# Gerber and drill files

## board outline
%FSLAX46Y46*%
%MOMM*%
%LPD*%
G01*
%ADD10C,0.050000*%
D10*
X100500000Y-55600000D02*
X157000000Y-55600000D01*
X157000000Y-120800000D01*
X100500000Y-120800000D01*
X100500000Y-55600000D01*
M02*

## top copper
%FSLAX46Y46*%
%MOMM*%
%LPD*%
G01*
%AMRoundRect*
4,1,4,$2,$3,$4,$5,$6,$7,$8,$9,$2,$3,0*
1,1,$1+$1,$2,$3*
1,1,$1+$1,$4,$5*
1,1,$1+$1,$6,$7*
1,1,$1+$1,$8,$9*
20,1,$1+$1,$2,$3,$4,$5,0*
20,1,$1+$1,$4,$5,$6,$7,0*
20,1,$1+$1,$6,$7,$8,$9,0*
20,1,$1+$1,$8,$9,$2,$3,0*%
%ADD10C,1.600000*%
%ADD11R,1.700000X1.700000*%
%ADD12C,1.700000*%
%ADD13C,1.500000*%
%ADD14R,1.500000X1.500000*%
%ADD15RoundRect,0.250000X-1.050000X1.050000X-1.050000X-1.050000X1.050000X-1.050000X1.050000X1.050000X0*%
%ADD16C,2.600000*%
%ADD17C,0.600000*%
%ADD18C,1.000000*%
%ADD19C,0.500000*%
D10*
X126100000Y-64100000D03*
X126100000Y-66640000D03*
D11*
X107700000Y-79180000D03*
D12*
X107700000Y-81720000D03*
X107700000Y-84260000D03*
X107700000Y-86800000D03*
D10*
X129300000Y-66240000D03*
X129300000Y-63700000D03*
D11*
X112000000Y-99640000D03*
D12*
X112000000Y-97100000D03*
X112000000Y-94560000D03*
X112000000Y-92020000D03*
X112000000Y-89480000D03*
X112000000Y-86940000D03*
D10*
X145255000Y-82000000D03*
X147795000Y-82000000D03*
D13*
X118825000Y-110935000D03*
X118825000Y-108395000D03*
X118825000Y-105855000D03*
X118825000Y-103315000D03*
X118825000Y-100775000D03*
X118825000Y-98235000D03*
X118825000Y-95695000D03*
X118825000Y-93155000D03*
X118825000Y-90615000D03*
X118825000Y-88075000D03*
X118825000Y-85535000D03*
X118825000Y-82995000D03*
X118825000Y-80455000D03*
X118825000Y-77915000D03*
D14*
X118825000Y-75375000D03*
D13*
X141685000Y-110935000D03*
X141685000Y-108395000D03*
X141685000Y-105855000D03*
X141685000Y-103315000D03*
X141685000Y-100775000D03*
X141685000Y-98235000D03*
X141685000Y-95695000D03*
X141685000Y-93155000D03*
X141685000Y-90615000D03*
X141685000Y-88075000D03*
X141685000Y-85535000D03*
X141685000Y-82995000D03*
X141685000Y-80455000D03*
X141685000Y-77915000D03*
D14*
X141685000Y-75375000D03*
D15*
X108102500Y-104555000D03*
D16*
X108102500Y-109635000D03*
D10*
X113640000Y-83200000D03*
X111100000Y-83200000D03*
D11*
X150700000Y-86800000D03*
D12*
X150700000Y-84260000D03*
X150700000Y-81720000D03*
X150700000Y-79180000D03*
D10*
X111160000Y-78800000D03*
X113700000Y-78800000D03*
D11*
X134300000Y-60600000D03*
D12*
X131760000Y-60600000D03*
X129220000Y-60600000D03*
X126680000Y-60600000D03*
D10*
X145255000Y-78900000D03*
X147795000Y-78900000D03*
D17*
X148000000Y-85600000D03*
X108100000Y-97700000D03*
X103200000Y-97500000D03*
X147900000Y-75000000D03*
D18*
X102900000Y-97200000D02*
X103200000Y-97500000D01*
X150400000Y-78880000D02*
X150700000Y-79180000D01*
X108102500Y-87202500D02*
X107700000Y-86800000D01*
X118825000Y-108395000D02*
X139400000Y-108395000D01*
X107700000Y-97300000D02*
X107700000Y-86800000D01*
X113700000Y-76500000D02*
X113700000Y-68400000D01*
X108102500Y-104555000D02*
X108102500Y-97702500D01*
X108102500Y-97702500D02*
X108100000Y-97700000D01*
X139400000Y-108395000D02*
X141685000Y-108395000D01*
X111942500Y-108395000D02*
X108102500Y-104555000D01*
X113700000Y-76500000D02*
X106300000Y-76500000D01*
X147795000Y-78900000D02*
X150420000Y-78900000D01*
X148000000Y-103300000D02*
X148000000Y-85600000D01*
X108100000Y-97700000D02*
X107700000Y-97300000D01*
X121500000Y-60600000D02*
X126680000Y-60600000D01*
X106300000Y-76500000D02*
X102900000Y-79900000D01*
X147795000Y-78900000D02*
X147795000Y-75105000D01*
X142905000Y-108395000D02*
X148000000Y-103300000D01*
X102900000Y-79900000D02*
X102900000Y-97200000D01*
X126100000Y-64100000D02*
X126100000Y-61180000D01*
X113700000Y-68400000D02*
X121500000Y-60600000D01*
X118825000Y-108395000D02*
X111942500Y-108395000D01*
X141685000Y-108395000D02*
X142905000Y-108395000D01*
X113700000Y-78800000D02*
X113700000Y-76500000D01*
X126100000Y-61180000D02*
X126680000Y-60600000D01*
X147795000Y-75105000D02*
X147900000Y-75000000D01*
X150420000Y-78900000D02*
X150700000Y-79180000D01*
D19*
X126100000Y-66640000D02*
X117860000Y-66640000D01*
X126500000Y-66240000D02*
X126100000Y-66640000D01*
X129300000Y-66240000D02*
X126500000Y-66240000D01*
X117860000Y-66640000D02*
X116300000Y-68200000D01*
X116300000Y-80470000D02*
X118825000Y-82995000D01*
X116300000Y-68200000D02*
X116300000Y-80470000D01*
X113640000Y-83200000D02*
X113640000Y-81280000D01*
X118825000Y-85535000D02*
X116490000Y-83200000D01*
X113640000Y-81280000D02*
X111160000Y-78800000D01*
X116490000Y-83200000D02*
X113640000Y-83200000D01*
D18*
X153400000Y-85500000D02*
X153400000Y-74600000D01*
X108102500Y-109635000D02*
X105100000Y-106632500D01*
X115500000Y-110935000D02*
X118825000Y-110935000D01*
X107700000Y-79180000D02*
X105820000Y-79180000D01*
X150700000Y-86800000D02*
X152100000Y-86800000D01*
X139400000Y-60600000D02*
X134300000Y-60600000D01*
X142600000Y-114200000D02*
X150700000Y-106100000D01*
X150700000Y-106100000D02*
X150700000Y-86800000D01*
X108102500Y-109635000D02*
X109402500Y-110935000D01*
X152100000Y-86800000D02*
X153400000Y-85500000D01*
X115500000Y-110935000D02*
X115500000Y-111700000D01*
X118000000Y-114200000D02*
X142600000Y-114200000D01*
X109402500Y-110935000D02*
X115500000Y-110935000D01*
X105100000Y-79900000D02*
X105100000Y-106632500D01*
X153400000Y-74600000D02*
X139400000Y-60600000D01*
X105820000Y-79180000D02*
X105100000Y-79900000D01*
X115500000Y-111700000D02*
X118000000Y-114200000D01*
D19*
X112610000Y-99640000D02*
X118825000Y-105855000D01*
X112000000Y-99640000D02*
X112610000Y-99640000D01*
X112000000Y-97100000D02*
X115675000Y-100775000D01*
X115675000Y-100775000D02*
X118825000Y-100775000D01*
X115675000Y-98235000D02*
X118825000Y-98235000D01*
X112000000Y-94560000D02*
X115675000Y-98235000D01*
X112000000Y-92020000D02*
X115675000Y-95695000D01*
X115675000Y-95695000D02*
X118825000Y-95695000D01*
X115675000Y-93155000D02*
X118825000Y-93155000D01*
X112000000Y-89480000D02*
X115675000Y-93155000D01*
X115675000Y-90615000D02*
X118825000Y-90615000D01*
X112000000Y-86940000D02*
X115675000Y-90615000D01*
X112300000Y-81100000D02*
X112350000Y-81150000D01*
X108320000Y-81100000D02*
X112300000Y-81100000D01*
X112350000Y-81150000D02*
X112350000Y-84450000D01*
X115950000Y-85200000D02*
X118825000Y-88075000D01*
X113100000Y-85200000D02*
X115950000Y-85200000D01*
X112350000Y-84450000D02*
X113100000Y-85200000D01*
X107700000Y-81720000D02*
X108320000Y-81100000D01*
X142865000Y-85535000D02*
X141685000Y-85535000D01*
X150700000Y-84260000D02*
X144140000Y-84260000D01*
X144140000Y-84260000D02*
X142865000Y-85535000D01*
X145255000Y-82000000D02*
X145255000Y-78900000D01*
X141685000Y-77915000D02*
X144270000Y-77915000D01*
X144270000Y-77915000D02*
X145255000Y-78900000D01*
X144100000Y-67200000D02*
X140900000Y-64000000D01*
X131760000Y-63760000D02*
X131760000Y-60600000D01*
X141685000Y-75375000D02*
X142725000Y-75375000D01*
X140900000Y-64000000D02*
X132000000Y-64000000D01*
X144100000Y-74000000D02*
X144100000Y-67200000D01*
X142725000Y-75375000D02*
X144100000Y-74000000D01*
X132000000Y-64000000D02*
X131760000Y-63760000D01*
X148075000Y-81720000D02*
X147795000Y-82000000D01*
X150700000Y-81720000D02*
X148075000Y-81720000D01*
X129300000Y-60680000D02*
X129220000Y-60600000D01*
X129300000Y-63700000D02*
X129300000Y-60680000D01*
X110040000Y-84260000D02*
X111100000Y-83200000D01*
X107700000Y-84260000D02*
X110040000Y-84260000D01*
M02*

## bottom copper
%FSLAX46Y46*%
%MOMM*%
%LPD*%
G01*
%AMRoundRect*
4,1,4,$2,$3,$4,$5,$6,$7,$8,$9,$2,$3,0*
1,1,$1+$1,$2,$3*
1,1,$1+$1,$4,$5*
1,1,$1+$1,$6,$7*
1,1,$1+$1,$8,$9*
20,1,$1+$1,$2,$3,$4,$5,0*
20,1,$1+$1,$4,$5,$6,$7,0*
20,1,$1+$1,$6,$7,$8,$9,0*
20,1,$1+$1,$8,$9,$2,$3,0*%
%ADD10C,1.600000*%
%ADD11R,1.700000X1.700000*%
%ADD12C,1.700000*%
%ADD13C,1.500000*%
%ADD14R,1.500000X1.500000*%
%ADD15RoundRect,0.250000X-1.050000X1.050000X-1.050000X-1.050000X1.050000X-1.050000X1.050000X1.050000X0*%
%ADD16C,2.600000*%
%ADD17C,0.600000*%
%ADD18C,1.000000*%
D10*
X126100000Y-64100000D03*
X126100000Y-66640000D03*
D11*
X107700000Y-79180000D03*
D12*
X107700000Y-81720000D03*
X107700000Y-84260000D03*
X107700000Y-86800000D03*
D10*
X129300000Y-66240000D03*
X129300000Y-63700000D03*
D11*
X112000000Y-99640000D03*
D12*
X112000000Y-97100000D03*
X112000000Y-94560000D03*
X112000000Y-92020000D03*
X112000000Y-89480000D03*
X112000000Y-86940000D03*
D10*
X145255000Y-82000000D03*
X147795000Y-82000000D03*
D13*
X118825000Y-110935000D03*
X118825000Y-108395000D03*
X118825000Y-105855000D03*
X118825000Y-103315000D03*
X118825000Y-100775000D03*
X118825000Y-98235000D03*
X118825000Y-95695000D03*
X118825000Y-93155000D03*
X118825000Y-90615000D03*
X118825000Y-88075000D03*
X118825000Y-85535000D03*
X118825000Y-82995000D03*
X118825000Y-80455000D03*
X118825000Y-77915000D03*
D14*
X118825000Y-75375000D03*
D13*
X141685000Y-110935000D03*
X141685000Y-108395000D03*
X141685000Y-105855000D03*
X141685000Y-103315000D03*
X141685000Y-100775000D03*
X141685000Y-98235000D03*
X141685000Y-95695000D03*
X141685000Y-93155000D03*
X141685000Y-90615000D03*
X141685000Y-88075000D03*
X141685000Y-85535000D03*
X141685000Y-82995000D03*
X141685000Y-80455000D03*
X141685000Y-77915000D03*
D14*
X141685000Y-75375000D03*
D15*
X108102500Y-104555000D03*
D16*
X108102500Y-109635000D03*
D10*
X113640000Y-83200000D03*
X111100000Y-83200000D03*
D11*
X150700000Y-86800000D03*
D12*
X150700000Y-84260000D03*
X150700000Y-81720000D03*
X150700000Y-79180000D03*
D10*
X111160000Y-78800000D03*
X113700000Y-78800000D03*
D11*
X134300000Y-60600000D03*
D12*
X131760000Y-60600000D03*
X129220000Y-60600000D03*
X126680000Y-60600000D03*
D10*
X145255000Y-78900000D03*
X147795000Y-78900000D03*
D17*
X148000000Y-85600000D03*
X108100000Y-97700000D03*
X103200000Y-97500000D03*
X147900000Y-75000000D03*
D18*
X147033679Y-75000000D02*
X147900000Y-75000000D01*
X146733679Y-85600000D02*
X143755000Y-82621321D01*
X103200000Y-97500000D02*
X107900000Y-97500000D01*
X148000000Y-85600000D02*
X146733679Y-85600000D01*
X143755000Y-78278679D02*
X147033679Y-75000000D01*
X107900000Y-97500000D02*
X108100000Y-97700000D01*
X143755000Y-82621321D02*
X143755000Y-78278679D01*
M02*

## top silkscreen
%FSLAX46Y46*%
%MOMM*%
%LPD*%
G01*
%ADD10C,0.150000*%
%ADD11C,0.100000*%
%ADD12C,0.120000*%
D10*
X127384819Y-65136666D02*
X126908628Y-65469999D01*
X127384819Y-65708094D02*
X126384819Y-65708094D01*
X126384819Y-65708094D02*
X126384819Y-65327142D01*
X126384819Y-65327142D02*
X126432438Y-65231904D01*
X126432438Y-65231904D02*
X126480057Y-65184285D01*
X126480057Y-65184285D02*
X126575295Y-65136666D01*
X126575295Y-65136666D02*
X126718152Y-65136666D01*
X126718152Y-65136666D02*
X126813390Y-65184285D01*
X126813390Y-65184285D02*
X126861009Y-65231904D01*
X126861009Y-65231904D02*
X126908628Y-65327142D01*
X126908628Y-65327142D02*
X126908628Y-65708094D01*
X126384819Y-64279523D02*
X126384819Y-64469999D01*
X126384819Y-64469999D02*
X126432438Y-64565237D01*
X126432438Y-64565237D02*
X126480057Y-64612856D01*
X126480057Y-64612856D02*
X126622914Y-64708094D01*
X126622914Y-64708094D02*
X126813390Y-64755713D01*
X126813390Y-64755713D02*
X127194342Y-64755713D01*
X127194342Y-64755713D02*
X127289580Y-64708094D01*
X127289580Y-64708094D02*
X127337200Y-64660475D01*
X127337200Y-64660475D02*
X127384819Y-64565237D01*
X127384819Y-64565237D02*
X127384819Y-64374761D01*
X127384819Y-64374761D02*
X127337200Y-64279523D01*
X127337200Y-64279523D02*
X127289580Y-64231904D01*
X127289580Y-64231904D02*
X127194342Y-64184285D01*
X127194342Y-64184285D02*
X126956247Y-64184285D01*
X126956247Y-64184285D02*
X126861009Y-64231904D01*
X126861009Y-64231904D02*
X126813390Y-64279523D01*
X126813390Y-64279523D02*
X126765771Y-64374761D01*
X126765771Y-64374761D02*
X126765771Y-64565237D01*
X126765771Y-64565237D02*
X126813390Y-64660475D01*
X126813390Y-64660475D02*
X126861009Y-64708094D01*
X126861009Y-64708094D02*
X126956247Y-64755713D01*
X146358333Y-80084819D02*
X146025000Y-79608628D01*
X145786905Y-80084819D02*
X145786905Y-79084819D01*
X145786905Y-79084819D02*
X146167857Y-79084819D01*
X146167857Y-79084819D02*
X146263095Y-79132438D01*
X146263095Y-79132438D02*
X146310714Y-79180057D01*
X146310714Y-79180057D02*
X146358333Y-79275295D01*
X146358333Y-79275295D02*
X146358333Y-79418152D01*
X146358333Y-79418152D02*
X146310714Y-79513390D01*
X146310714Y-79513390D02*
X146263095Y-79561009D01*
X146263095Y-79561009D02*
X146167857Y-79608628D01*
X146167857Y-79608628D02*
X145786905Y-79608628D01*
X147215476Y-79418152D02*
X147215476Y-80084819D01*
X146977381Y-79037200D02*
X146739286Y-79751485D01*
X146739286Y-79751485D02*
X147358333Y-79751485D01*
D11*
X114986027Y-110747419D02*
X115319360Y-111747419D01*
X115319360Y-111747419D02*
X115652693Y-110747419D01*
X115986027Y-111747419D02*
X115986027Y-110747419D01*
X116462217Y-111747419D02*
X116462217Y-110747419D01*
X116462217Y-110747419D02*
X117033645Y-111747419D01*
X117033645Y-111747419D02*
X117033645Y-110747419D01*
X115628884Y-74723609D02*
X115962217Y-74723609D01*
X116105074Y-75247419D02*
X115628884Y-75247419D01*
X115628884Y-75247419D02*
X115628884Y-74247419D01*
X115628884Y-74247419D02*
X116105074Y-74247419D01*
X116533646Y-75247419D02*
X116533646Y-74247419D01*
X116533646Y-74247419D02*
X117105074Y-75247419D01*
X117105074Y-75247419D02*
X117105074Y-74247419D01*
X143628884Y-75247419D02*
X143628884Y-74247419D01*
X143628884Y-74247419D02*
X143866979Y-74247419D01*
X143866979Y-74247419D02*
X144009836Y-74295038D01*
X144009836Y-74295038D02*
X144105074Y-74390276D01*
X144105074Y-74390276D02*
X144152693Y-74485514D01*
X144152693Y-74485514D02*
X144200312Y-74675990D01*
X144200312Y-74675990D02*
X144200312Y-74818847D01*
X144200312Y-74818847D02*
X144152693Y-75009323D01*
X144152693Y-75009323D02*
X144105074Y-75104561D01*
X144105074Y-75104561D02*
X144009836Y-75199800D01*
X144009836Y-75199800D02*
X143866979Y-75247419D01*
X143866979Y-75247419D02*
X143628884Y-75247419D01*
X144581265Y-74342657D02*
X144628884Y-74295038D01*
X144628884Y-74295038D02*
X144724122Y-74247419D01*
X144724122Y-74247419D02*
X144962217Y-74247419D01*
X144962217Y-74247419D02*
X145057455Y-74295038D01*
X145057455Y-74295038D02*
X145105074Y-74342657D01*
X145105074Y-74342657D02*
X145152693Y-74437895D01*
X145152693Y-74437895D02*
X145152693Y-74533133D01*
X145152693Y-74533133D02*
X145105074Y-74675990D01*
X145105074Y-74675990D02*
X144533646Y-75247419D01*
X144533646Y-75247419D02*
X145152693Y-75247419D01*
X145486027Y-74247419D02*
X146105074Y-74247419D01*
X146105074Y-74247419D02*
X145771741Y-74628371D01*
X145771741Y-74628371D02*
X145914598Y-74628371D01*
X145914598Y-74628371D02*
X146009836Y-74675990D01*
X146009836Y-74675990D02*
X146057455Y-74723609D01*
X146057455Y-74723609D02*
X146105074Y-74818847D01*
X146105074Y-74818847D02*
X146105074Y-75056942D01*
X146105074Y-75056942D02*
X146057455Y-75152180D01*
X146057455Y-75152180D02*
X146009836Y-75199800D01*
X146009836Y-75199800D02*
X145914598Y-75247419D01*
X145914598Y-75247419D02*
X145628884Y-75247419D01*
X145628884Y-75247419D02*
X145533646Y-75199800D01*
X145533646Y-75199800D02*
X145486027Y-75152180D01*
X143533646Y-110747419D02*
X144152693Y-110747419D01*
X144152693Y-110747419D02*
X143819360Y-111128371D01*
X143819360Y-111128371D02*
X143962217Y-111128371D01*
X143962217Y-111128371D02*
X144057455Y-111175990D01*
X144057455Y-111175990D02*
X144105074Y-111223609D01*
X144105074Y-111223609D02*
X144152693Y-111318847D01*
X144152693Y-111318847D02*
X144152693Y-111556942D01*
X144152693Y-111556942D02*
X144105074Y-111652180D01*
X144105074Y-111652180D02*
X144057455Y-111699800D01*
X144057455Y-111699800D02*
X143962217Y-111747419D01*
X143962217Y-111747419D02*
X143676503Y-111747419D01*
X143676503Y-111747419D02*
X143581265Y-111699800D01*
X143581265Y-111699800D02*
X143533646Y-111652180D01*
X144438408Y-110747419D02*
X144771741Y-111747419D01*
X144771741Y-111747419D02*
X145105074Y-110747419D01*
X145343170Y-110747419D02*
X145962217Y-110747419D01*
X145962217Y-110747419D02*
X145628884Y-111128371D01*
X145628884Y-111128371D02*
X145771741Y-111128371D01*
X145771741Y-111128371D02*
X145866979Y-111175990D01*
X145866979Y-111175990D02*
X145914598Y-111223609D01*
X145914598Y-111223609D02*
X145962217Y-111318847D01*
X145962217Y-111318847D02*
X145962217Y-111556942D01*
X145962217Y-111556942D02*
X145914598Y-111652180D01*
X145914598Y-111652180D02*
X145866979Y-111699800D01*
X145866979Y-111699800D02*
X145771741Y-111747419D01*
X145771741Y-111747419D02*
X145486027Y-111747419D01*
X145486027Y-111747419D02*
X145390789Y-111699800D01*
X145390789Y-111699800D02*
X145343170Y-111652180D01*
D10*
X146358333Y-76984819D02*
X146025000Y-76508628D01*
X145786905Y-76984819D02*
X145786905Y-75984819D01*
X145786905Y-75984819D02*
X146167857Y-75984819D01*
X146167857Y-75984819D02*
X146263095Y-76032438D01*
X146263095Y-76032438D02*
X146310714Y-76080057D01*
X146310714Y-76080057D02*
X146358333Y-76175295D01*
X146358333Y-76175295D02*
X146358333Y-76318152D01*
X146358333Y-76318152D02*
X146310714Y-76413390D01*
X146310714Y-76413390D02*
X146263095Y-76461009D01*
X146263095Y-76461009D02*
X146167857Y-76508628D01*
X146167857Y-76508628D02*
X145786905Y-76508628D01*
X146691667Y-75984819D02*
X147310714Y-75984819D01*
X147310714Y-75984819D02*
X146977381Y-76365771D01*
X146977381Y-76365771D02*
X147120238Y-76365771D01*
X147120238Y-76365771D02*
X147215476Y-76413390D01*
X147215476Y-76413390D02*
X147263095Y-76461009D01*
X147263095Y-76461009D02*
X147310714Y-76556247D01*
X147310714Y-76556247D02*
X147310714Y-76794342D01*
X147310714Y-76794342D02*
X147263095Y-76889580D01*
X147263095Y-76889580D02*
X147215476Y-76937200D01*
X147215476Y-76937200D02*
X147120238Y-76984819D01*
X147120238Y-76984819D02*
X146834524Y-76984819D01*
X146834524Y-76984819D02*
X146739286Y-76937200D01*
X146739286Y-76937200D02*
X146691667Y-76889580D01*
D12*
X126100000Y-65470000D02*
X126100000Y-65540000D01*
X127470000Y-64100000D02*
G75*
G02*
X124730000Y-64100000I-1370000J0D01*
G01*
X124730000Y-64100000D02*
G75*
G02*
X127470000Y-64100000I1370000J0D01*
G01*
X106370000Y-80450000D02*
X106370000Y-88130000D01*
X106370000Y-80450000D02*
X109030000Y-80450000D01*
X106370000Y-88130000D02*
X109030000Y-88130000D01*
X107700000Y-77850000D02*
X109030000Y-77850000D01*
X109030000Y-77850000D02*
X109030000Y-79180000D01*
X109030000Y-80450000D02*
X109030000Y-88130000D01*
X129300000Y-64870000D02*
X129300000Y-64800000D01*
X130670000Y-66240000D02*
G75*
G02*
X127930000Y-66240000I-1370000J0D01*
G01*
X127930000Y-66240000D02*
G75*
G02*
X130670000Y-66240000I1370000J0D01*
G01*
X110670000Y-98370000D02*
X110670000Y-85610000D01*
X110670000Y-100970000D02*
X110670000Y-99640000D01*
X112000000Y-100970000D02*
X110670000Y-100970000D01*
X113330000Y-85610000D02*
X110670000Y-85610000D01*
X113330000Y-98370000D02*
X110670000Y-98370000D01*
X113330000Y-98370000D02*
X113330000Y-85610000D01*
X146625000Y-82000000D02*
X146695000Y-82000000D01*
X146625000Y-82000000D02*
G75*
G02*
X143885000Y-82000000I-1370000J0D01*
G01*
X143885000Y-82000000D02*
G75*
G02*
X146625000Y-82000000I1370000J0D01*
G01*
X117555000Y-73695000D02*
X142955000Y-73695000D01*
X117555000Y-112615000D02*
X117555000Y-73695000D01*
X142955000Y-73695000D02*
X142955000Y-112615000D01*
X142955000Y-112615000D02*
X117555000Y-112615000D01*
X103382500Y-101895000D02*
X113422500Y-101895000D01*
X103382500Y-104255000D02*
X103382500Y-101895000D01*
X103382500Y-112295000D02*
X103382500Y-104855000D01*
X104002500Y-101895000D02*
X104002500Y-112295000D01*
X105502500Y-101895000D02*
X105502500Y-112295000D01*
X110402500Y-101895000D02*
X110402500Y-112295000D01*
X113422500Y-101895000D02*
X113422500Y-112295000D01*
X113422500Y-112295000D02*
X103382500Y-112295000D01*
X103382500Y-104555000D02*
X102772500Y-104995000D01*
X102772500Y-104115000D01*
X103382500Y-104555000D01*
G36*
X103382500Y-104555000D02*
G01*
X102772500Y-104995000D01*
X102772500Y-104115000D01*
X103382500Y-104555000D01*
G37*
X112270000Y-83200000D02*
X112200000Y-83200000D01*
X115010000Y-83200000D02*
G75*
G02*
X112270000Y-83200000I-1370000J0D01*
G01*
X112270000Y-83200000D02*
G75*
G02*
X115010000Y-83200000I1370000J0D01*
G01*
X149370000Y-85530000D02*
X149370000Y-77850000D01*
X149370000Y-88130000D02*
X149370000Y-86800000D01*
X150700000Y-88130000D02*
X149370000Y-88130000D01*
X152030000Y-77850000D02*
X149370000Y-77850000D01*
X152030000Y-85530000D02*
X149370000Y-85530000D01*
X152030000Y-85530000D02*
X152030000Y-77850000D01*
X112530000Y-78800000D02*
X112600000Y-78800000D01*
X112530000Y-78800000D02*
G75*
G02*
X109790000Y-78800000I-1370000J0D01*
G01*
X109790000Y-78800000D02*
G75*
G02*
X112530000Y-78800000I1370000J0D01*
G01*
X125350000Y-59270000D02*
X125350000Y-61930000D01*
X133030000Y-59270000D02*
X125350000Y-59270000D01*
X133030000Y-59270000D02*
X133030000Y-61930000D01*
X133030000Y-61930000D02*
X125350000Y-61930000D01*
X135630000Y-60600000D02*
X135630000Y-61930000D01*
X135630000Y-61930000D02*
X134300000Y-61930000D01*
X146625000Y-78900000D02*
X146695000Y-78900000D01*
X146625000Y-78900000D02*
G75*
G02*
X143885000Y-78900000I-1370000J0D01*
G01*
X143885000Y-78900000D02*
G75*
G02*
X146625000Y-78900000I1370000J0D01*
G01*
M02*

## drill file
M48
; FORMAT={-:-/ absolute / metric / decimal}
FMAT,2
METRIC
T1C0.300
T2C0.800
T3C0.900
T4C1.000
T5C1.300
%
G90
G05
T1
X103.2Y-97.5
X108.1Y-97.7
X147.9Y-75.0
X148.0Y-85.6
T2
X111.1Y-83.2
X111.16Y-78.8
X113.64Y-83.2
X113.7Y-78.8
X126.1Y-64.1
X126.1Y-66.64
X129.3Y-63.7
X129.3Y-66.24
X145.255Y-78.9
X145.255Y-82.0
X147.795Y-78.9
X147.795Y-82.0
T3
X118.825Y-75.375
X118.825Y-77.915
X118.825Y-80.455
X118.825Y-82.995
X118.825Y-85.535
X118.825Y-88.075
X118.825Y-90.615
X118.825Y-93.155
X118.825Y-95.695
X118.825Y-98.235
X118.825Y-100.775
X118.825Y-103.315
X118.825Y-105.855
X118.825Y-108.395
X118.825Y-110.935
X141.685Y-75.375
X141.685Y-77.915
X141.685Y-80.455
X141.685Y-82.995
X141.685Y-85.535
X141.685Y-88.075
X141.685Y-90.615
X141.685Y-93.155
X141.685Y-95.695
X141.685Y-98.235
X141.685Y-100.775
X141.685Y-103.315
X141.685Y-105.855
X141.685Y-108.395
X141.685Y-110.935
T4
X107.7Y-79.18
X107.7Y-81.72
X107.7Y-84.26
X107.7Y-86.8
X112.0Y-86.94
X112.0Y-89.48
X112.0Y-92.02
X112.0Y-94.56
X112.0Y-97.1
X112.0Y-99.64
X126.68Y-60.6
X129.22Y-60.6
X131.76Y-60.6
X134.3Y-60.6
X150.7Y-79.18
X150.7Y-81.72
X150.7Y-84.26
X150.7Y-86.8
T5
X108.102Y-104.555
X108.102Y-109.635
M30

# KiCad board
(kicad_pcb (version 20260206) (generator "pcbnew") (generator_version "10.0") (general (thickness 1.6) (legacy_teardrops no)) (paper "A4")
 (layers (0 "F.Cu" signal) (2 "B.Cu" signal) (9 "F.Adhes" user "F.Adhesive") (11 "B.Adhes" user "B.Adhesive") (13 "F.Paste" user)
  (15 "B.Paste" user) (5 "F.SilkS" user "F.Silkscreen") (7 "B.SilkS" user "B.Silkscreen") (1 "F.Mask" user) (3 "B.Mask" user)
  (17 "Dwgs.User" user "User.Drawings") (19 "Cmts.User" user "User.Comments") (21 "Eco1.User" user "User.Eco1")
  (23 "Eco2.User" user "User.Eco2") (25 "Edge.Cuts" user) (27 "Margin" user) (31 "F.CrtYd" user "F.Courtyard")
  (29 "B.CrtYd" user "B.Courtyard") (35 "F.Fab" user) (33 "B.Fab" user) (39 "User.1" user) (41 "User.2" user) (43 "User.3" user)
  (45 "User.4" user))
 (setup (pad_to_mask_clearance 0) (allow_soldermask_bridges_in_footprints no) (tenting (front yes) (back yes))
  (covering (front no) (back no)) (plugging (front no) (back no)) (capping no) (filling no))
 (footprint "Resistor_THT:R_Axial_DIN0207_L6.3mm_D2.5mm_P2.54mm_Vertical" (layer "F.Cu") (at 126.1 64.1 -90)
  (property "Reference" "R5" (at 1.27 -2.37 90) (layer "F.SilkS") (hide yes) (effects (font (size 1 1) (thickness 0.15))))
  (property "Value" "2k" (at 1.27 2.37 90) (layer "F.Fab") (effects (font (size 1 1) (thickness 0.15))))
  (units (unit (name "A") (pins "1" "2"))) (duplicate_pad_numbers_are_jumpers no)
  (fp_line (start 1.37 0) (end 1.44 0) (stroke (width 0.12) (type solid)) (layer "F.SilkS"))
  (fp_circle (center 0 0) (end 1.37 0) (stroke (width 0.12) (type solid)) (fill no) (layer "F.SilkS"))
  (pad "1" thru_hole circle (at 0 0 270) (size 1.6 1.6) (drill 0.8) (layers "*.Cu" "*.Mask") (remove_unused_layers no) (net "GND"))
  (pad "2" thru_hole circle (at 2.54 0 270) (size 1.6 1.6) (drill 0.8) (layers "*.Cu" "*.Mask") (remove_unused_layers no)
   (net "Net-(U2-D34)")))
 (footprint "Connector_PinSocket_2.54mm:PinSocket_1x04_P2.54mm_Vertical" (layer "F.Cu") (at 107.7 79.18)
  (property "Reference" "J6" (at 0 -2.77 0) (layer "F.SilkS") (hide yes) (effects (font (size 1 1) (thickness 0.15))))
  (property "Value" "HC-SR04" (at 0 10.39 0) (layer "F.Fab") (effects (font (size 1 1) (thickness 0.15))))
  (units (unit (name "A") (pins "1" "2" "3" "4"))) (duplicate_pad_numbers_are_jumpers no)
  (fp_line (start -1.33 1.27) (end -1.33 8.95) (stroke (width 0.12) (type solid)) (layer "F.SilkS"))
  (fp_line (start -1.33 1.27) (end 1.33 1.27) (stroke (width 0.12) (type solid)) (layer "F.SilkS"))
  (fp_line (start -1.33 8.95) (end 1.33 8.95) (stroke (width 0.12) (type solid)) (layer "F.SilkS"))
  (fp_line (start 0 -1.33) (end 1.33 -1.33) (stroke (width 0.12) (type solid)) (layer "F.SilkS"))
  (fp_line (start 1.33 -1.33) (end 1.33 0) (stroke (width 0.12) (type solid)) (layer "F.SilkS"))
  (fp_line (start 1.33 1.27) (end 1.33 8.95) (stroke (width 0.12) (type solid)) (layer "F.SilkS"))
  (pad "1" thru_hole rect (at 0 0) (size 1.7 1.7) (drill 1) (layers "*.Cu" "*.Mask") (remove_unused_layers no) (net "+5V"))
  (pad "2" thru_hole circle (at 0 2.54) (size 1.7 1.7) (drill 1) (layers "*.Cu" "*.Mask") (remove_unused_layers no) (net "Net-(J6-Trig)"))
  (pad "3" thru_hole circle (at 0 5.08) (size 1.7 1.7) (drill 1) (layers "*.Cu" "*.Mask") (remove_unused_layers no) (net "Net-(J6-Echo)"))
  (pad "4" thru_hole circle (at 0 7.62) (size 1.7 1.7) (drill 1) (layers "*.Cu" "*.Mask") (remove_unused_layers no) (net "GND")))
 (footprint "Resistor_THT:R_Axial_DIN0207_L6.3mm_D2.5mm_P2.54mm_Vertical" (layer "F.Cu") (at 129.3 66.24 90)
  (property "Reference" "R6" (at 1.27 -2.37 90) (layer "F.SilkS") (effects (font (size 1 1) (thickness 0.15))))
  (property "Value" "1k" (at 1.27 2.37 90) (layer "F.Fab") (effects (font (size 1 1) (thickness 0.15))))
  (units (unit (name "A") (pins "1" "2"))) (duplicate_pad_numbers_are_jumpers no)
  (fp_line (start 1.37 0) (end 1.44 0) (stroke (width 0.12) (type solid)) (layer "F.SilkS"))
  (fp_circle (center 0 0) (end 1.37 0) (stroke (width 0.12) (type solid)) (fill no) (layer "F.SilkS"))
  (pad "1" thru_hole circle (at 0 0 90) (size 1.6 1.6) (drill 0.8) (layers "*.Cu" "*.Mask") (remove_unused_layers no) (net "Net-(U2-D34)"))
  (pad "2" thru_hole circle (at 2.54 0 90) (size 1.6 1.6) (drill 0.8) (layers "*.Cu" "*.Mask") (remove_unused_layers no)
   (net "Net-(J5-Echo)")))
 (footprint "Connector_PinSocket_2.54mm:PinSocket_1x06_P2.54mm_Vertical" (layer "F.Cu") (at 112 99.64 180)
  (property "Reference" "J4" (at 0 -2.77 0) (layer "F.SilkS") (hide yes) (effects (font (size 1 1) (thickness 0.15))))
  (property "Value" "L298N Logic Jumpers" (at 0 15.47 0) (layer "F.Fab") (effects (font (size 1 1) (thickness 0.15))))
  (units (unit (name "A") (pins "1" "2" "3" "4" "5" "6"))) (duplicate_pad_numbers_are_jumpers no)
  (fp_line (start 1.33 1.27) (end 1.33 14.03) (stroke (width 0.12) (type solid)) (layer "F.SilkS"))
  (fp_line (start 1.33 -1.33) (end 1.33 0) (stroke (width 0.12) (type solid)) (layer "F.SilkS"))
  (fp_line (start 0 -1.33) (end 1.33 -1.33) (stroke (width 0.12) (type solid)) (layer "F.SilkS"))
  (fp_line (start -1.33 14.03) (end 1.33 14.03) (stroke (width 0.12) (type solid)) (layer "F.SilkS"))
  (fp_line (start -1.33 1.27) (end 1.33 1.27) (stroke (width 0.12) (type solid)) (layer "F.SilkS"))
  (fp_line (start -1.33 1.27) (end -1.33 14.03) (stroke (width 0.12) (type solid)) (layer "F.SilkS"))
  (pad "1" thru_hole rect (at 0 0 180) (size 1.7 1.7) (drill 1) (layers "*.Cu" "*.Mask") (remove_unused_layers no) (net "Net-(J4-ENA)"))
  (pad "2" thru_hole circle (at 0 2.54 180) (size 1.7 1.7) (drill 1) (layers "*.Cu" "*.Mask") (remove_unused_layers no)
   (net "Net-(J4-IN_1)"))
  (pad "3" thru_hole circle (at 0 5.08 180) (size 1.7 1.7) (drill 1) (layers "*.Cu" "*.Mask") (remove_unused_layers no)
   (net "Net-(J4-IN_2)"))
  (pad "4" thru_hole circle (at 0 7.62 180) (size 1.7 1.7) (drill 1) (layers "*.Cu" "*.Mask") (remove_unused_layers no)
   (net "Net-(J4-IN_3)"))
  (pad "5" thru_hole circle (at 0 10.16 180) (size 1.7 1.7) (drill 1) (layers "*.Cu" "*.Mask") (remove_unused_layers no)
   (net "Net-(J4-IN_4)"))
  (pad "6" thru_hole circle (at 0 12.7 180) (size 1.7 1.7) (drill 1) (layers "*.Cu" "*.Mask") (remove_unused_layers no) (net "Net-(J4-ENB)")))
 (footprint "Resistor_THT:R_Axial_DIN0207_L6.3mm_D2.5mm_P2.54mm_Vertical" (layer "F.Cu") (at 145.255 82)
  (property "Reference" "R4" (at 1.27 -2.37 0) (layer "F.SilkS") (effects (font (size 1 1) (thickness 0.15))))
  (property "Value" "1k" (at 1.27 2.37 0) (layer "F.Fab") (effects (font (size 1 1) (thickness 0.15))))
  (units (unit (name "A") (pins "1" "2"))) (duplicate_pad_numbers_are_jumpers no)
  (fp_line (start 1.37 0) (end 1.44 0) (stroke (width 0.12) (type solid)) (layer "F.SilkS"))
  (fp_circle (center 0 0) (end 1.37 0) (stroke (width 0.12) (type solid)) (fill no) (layer "F.SilkS"))
  (pad "1" thru_hole circle (at 0 0) (size 1.6 1.6) (drill 0.8) (layers "*.Cu" "*.Mask") (remove_unused_layers no) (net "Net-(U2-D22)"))
  (pad "2" thru_hole circle (at 2.54 0) (size 1.6 1.6) (drill 0.8) (layers "*.Cu" "*.Mask") (remove_unused_layers no) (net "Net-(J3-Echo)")))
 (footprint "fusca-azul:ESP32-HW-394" (layer "F.Cu") (at 118.825 75.375)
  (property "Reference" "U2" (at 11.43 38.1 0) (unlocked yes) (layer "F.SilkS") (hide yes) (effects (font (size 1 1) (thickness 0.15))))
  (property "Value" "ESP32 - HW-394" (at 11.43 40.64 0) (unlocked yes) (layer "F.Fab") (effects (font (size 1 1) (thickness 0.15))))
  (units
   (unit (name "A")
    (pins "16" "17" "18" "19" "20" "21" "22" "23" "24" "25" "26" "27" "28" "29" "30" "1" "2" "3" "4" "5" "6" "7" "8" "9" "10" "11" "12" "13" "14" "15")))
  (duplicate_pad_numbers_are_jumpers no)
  (fp_line (start -1.27 -1.68) (end 24.13 -1.68) (stroke (width 0.12) (type solid)) (layer "F.SilkS"))
  (fp_line (start -1.27 37.24) (end -1.27 -1.68) (stroke (width 0.12) (type solid)) (layer "F.SilkS"))
  (fp_line (start 24.13 -1.68) (end 24.13 37.24) (stroke (width 0.12) (type solid)) (layer "F.SilkS"))
  (fp_line (start 24.13 37.24) (end -1.27 37.24) (stroke (width 0.12) (type solid)) (layer "F.SilkS"))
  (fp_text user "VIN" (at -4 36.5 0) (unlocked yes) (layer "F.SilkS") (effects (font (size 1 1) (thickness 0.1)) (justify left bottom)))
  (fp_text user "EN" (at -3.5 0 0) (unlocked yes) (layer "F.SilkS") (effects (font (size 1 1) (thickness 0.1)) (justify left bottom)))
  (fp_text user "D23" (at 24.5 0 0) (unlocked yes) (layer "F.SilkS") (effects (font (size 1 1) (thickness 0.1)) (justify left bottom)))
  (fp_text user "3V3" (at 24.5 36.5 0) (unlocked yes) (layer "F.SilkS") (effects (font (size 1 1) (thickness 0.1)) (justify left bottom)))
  (pad "1" thru_hole circle (at 0 35.56 180) (size 1.5 1.5) (drill 0.9) (layers "*.Cu" "*.Mask") (remove_unused_layers yes)
   (keep_end_layers yes) (zone_layer_connections) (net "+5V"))
  (pad "2" thru_hole circle (at 0 33.02 180) (size 1.5 1.5) (drill 0.9) (layers "*.Cu" "*.Mask") (remove_unused_layers yes)
   (keep_end_layers yes) (zone_layer_connections) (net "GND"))
  (pad "3" thru_hole circle (at 0 30.48 180) (size 1.5 1.5) (drill 0.9) (layers "*.Cu" "*.Mask") (remove_unused_layers yes)
   (keep_end_layers yes) (zone_layer_connections) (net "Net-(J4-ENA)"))
  (pad "4" thru_hole circle (at 0 27.94 180) (size 1.5 1.5) (drill 0.9) (layers "*.Cu" "*.Mask") (remove_unused_layers yes)
   (keep_end_layers yes) (zone_layer_connections) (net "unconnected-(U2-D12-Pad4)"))
  (pad "5" thru_hole circle (at 0 25.4 180) (size 1.5 1.5) (drill 0.9) (layers "*.Cu" "*.Mask") (remove_unused_layers yes)
   (keep_end_layers yes) (zone_layer_connections) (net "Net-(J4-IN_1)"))
  (pad "6" thru_hole circle (at 0 22.86 180) (size 1.5 1.5) (drill 0.9) (layers "*.Cu" "*.Mask") (remove_unused_layers yes)
   (keep_end_layers yes) (zone_layer_connections) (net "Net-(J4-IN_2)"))
  (pad "7" thru_hole circle (at 0 20.32 180) (size 1.5 1.5) (drill 0.9) (layers "*.Cu" "*.Mask") (remove_unused_layers yes)
   (keep_end_layers yes) (zone_layer_connections) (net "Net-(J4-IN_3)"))
  (pad "8" thru_hole circle (at 0 17.78 180) (size 1.5 1.5) (drill 0.9) (layers "*.Cu" "*.Mask") (remove_unused_layers yes)
   (keep_end_layers yes) (zone_layer_connections) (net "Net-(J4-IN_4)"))
  (pad "9" thru_hole circle (at 0 15.24 180) (size 1.5 1.5) (drill 0.9) (layers "*.Cu" "*.Mask") (remove_unused_layers yes)
   (keep_end_layers yes) (zone_layer_connections) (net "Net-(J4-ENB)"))
  (pad "10" thru_hole circle (at 0 12.7 180) (size 1.5 1.5) (drill 0.9) (layers "*.Cu" "*.Mask") (remove_unused_layers yes)
   (keep_end_layers yes) (zone_layer_connections) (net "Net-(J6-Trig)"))
  (pad "11" thru_hole circle (at 0 10.16 180) (size 1.5 1.5) (drill 0.9) (layers "*.Cu" "*.Mask") (remove_unused_layers yes)
   (keep_end_layers yes) (zone_layer_connections) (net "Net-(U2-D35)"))
  (pad "12" thru_hole circle (at 0 7.62 180) (size 1.5 1.5) (drill 0.9) (layers "*.Cu" "*.Mask") (remove_unused_layers yes)
   (keep_end_layers yes) (zone_layer_connections) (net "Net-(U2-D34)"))
  (pad "13" thru_hole circle (at 0 5.08 180) (size 1.5 1.5) (drill 0.9) (layers "*.Cu" "*.Mask") (remove_unused_layers yes)
   (keep_end_layers yes) (zone_layer_connections) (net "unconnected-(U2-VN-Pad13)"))
  (pad "14" thru_hole circle (at 0 2.54 180) (size 1.5 1.5) (drill 0.9) (layers "*.Cu" "*.Mask") (remove_unused_layers yes)
   (keep_end_layers yes) (zone_layer_connections) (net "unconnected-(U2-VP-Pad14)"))
  (pad "15" thru_hole rect (at 0 0 180) (size 1.5 1.5) (drill 0.9) (layers "*.Cu" "*.Mask") (remove_unused_layers yes) (keep_end_layers yes)
   (zone_layer_connections) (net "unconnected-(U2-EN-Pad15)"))
  (pad "16" thru_hole circle (at 22.86 35.56) (size 1.5 1.5) (drill 0.9) (layers "*.Cu" "*.Mask") (remove_unused_layers yes)
   (keep_end_layers yes) (zone_layer_connections) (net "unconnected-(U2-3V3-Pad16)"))
  (pad "17" thru_hole circle (at 22.86 33.02) (size 1.5 1.5) (drill 0.9) (layers "*.Cu" "*.Mask") (remove_unused_layers yes)
   (keep_end_layers yes) (zone_layer_connections) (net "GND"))
  (pad "18" thru_hole circle (at 22.86 30.48) (size 1.5 1.5) (drill 0.9) (layers "*.Cu" "*.Mask") (remove_unused_layers yes)
   (keep_end_layers yes) (zone_layer_connections) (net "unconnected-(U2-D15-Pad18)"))
  (pad "19" thru_hole circle (at 22.86 27.94) (size 1.5 1.5) (drill 0.9) (layers "*.Cu" "*.Mask") (remove_unused_layers yes)
   (keep_end_layers yes) (zone_layer_connections) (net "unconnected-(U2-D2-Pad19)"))
  (pad "20" thru_hole circle (at 22.86 25.4) (size 1.5 1.5) (drill 0.9) (layers "*.Cu" "*.Mask") (remove_unused_layers yes)
   (keep_end_layers yes) (zone_layer_connections) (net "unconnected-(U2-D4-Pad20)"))
  (pad "21" thru_hole circle (at 22.86 22.86) (size 1.5 1.5) (drill 0.9) (layers "*.Cu" "*.Mask") (remove_unused_layers yes)
   (keep_end_layers yes) (zone_layer_connections) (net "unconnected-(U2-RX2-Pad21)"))
  (pad "22" thru_hole circle (at 22.86 20.32) (size 1.5 1.5) (drill 0.9) (layers "*.Cu" "*.Mask") (remove_unused_layers yes)
   (keep_end_layers yes) (zone_layer_connections) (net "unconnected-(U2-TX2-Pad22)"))
  (pad "23" thru_hole circle (at 22.86 17.78) (size 1.5 1.5) (drill 0.9) (layers "*.Cu" "*.Mask") (remove_unused_layers yes)
   (keep_end_layers yes) (zone_layer_connections) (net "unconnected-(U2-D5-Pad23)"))
  (pad "24" thru_hole circle (at 22.86 15.24) (size 1.5 1.5) (drill 0.9) (layers "*.Cu" "*.Mask") (remove_unused_layers yes)
   (keep_end_layers yes) (zone_layer_connections) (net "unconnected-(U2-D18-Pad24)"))
  (pad "25" thru_hole circle (at 22.86 12.7) (size 1.5 1.5) (drill 0.9) (layers "*.Cu" "*.Mask") (remove_unused_layers yes)
   (keep_end_layers yes) (zone_layer_connections) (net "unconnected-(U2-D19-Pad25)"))
  (pad "26" thru_hole circle (at 22.86 10.16) (size 1.5 1.5) (drill 0.9) (layers "*.Cu" "*.Mask") (remove_unused_layers yes)
   (keep_end_layers yes) (zone_layer_connections) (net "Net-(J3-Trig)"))
  (pad "27" thru_hole circle (at 22.86 7.62) (size 1.5 1.5) (drill 0.9) (layers "*.Cu" "*.Mask") (remove_unused_layers yes)
   (keep_end_layers yes) (zone_layer_connections) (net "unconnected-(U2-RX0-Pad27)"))
  (pad "28" thru_hole circle (at 22.86 5.08) (size 1.5 1.5) (drill 0.9) (layers "*.Cu" "*.Mask") (remove_unused_layers yes)
   (keep_end_layers yes) (zone_layer_connections) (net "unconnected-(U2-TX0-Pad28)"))
  (pad "29" thru_hole circle (at 22.86 2.54) (size 1.5 1.5) (drill 0.9) (layers "*.Cu" "*.Mask") (remove_unused_layers yes)
   (keep_end_layers yes) (zone_layer_connections) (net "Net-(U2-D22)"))
  (pad "30" thru_hole rect (at 22.86 0) (size 1.5 1.5) (drill 0.9) (layers "*.Cu" "*.Mask") (remove_unused_layers yes) (keep_end_layers yes)
   (zone_layer_connections) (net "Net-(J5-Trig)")))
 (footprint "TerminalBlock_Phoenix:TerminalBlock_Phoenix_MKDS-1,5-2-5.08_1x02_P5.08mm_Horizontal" (layer "F.Cu") (at 108.1025 104.555 -90)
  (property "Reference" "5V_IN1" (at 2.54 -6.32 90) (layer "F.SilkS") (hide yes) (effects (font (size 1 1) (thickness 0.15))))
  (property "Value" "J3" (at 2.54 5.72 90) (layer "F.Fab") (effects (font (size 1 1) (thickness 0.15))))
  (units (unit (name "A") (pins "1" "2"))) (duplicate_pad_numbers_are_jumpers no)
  (fp_line (start -2.66 4.72) (end -2.66 -5.32) (stroke (width 0.12) (type solid)) (layer "F.SilkS"))
  (fp_line (start -0.3 4.72) (end -2.66 4.72) (stroke (width 0.12) (type solid)) (layer "F.SilkS"))
  (fp_line (start 7.74 4.72) (end 0.3 4.72) (stroke (width 0.12) (type solid)) (layer "F.SilkS"))
  (fp_line (start -2.66 4.1) (end 7.74 4.1) (stroke (width 0.12) (type solid)) (layer "F.SilkS"))
  (fp_line (start -2.66 2.6) (end 7.74 2.6) (stroke (width 0.12) (type solid)) (layer "F.SilkS"))
  (fp_line (start -2.66 -2.3) (end 7.74 -2.3) (stroke (width 0.12) (type solid)) (layer "F.SilkS"))
  (fp_line (start -2.66 -5.32) (end 7.74 -5.32) (stroke (width 0.12) (type solid)) (layer "F.SilkS"))
  (fp_line (start 7.74 -5.32) (end 7.74 4.72) (stroke (width 0.12) (type solid)) (layer "F.SilkS"))
  (fp_poly (pts (xy 0 4.72) (xy 0.44 5.33) (xy -0.44 5.33)) (stroke (width 0.12) (type solid)) (fill yes) (layer "F.SilkS"))
  (pad "1" thru_hole roundrect (at 0 0 270) (size 2.6 2.6) (drill 1.3) (layers "*.Cu" "*.Mask") (remove_unused_layers no)
   (roundrect_rratio 0.096154) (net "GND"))
  (pad "2" thru_hole circle (at 5.08 0 270) (size 2.6 2.6) (drill 1.3) (layers "*.Cu" "*.Mask") (remove_unused_layers no) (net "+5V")))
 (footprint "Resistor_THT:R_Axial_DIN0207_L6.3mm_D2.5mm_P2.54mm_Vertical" (layer "F.Cu") (at 113.64 83.2 180)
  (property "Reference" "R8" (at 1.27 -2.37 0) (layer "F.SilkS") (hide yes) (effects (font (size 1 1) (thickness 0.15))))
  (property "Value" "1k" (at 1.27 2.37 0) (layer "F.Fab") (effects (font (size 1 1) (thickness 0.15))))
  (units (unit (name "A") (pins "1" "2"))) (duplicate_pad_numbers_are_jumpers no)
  (fp_line (start 1.37 0) (end 1.44 0) (stroke (width 0.12) (type solid)) (layer "F.SilkS"))
  (fp_circle (center 0 0) (end 1.37 0) (stroke (width 0.12) (type solid)) (fill no) (layer "F.SilkS"))
  (pad "1" thru_hole circle (at 0 0 180) (size 1.6 1.6) (drill 0.8) (layers "*.Cu" "*.Mask") (remove_unused_layers no) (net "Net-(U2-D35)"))
  (pad "2" thru_hole circle (at 2.54 0 180) (size 1.6 1.6) (drill 0.8) (layers "*.Cu" "*.Mask") (remove_unused_layers no)
   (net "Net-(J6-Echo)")))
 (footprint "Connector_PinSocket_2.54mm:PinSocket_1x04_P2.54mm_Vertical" (layer "F.Cu") (at 150.7 86.8 180)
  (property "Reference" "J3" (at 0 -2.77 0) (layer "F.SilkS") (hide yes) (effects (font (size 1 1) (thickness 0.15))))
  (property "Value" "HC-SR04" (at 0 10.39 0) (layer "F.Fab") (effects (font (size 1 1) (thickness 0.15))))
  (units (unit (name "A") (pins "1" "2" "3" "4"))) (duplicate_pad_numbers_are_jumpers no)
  (fp_line (start 1.33 1.27) (end 1.33 8.95) (stroke (width 0.12) (type solid)) (layer "F.SilkS"))
  (fp_line (start 1.33 -1.33) (end 1.33 0) (stroke (width 0.12) (type solid)) (layer "F.SilkS"))
  (fp_line (start 0 -1.33) (end 1.33 -1.33) (stroke (width 0.12) (type solid)) (layer "F.SilkS"))
  (fp_line (start -1.33 8.95) (end 1.33 8.95) (stroke (width 0.12) (type solid)) (layer "F.SilkS"))
  (fp_line (start -1.33 1.27) (end 1.33 1.27) (stroke (width 0.12) (type solid)) (layer "F.SilkS"))
  (fp_line (start -1.33 1.27) (end -1.33 8.95) (stroke (width 0.12) (type solid)) (layer "F.SilkS"))
  (pad "1" thru_hole rect (at 0 0 180) (size 1.7 1.7) (drill 1) (layers "*.Cu" "*.Mask") (remove_unused_layers no) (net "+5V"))
  (pad "2" thru_hole circle (at 0 2.54 180) (size 1.7 1.7) (drill 1) (layers "*.Cu" "*.Mask") (remove_unused_layers no)
   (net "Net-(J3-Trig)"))
  (pad "3" thru_hole circle (at 0 5.08 180) (size 1.7 1.7) (drill 1) (layers "*.Cu" "*.Mask") (remove_unused_layers no)
   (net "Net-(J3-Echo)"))
  (pad "4" thru_hole circle (at 0 7.62 180) (size 1.7 1.7) (drill 1) (layers "*.Cu" "*.Mask") (remove_unused_layers no) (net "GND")))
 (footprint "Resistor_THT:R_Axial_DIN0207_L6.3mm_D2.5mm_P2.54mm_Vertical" (layer "F.Cu") (at 111.16 78.8)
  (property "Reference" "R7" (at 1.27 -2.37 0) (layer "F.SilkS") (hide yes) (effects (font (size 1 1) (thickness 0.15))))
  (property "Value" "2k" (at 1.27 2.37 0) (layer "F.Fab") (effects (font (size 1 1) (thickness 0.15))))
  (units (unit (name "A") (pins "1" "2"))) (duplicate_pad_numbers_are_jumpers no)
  (fp_line (start 1.37 0) (end 1.44 0) (stroke (width 0.12) (type solid)) (layer "F.SilkS"))
  (fp_circle (center 0 0) (end 1.37 0) (stroke (width 0.12) (type solid)) (fill no) (layer "F.SilkS"))
  (pad "1" thru_hole circle (at 0 0) (size 1.6 1.6) (drill 0.8) (layers "*.Cu" "*.Mask") (remove_unused_layers no) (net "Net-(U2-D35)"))
  (pad "2" thru_hole circle (at 2.54 0) (size 1.6 1.6) (drill 0.8) (layers "*.Cu" "*.Mask") (remove_unused_layers no) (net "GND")))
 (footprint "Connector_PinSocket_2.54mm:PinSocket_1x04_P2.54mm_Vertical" (layer "F.Cu") (at 134.3 60.6 -90)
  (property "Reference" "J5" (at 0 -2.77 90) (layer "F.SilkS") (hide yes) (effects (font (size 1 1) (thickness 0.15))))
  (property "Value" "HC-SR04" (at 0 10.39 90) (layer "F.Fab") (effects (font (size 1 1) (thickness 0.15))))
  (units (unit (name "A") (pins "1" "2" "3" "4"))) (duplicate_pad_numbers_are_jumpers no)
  (fp_line (start -1.33 8.95) (end 1.33 8.95) (stroke (width 0.12) (type solid)) (layer "F.SilkS"))
  (fp_line (start -1.33 1.27) (end -1.33 8.95) (stroke (width 0.12) (type solid)) (layer "F.SilkS"))
  (fp_line (start -1.33 1.27) (end 1.33 1.27) (stroke (width 0.12) (type solid)) (layer "F.SilkS"))
  (fp_line (start 1.33 1.27) (end 1.33 8.95) (stroke (width 0.12) (type solid)) (layer "F.SilkS"))
  (fp_line (start 0 -1.33) (end 1.33 -1.33) (stroke (width 0.12) (type solid)) (layer "F.SilkS"))
  (fp_line (start 1.33 -1.33) (end 1.33 0) (stroke (width 0.12) (type solid)) (layer "F.SilkS"))
  (pad "1" thru_hole rect (at 0 0 270) (size 1.7 1.7) (drill 1) (layers "*.Cu" "*.Mask") (remove_unused_layers no) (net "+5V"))
  (pad "2" thru_hole circle (at 0 2.54 270) (size 1.7 1.7) (drill 1) (layers "*.Cu" "*.Mask") (remove_unused_layers no)
   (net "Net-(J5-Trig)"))
  (pad "3" thru_hole circle (at 0 5.08 270) (size 1.7 1.7) (drill 1) (layers "*.Cu" "*.Mask") (remove_unused_layers no)
   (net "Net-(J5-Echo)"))
  (pad "4" thru_hole circle (at 0 7.62 270) (size 1.7 1.7) (drill 1) (layers "*.Cu" "*.Mask") (remove_unused_layers no) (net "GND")))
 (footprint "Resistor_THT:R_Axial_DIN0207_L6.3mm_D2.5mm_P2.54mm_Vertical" (layer "F.Cu") (at 145.255 78.9)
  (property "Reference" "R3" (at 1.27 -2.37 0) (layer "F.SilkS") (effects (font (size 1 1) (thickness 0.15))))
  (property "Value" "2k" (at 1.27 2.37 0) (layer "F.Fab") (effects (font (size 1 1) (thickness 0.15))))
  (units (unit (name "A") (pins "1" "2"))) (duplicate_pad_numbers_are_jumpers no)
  (fp_line (start 1.37 0) (end 1.44 0) (stroke (width 0.12) (type solid)) (layer "F.SilkS"))
  (fp_circle (center 0 0) (end 1.37 0) (stroke (width 0.12) (type solid)) (fill no) (layer "F.SilkS"))
  (pad "1" thru_hole circle (at 0 0) (size 1.6 1.6) (drill 0.8) (layers "*.Cu" "*.Mask") (remove_unused_layers no) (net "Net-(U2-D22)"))
  (pad "2" thru_hole circle (at 2.54 0) (size 1.6 1.6) (drill 0.8) (layers "*.Cu" "*.Mask") (remove_unused_layers no) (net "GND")))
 (gr_rect (start 100.5 55.6) (end 157 120.8) (stroke (width 0.05) (type default)) (fill no) (layer "Edge.Cuts"))
 (segment (start 102.9 97.2) (end 103.2 97.5) (width 1) (layer "F.Cu") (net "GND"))
 (segment (start 150.4 78.88) (end 150.7 79.18) (width 1) (layer "F.Cu") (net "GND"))
 (segment (start 108.1025 87.2025) (end 107.7 86.8) (width 1) (layer "F.Cu") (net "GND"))
 (segment (start 118.825 108.395) (end 139.4 108.395) (width 1) (layer "F.Cu") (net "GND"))
 (segment (start 107.7 97.3) (end 107.7 86.8) (width 1) (layer "F.Cu") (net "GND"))
 (segment (start 113.7 76.5) (end 113.7 68.4) (width 1) (layer "F.Cu") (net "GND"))
 (segment (start 108.1025 104.555) (end 108.1025 97.7025) (width 1) (layer "F.Cu") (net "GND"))
 (segment (start 108.1025 97.7025) (end 108.1 97.7) (width 1) (layer "F.Cu") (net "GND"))
 (segment (start 139.4 108.395) (end 141.685 108.395) (width 1) (layer "F.Cu") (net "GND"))
 (segment (start 111.9425 108.395) (end 108.1025 104.555) (width 1) (layer "F.Cu") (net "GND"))
 (segment (start 113.7 76.5) (end 106.3 76.5) (width 1) (layer "F.Cu") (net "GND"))
 (segment (start 147.795 78.9) (end 150.42 78.9) (width 1) (layer "F.Cu") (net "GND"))
 (segment (start 148 103.3) (end 148 85.6) (width 1) (layer "F.Cu") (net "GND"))
 (segment (start 108.1 97.7) (end 107.7 97.3) (width 1) (layer "F.Cu") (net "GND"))
 (segment (start 121.5 60.6) (end 126.68 60.6) (width 1) (layer "F.Cu") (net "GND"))
 (segment (start 106.3 76.5) (end 102.9 79.9) (width 1) (layer "F.Cu") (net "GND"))
 (segment (start 147.795 78.9) (end 147.795 75.105) (width 1) (layer "F.Cu") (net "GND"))
 (segment (start 142.905 108.395) (end 148 103.3) (width 1) (layer "F.Cu") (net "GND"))
 (segment (start 102.9 79.9) (end 102.9 97.2) (width 1) (layer "F.Cu") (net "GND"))
 (segment (start 126.1 64.1) (end 126.1 61.18) (width 1) (layer "F.Cu") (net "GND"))
 (segment (start 113.7 68.4) (end 121.5 60.6) (width 1) (layer "F.Cu") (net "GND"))
 (segment (start 118.825 108.395) (end 111.9425 108.395) (width 1) (layer "F.Cu") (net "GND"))
 (segment (start 141.685 108.395) (end 142.905 108.395) (width 1) (layer "F.Cu") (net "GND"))
 (segment (start 113.7 78.8) (end 113.7 76.5) (width 1) (layer "F.Cu") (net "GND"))
 (segment (start 126.1 61.18) (end 126.68 60.6) (width 1) (layer "F.Cu") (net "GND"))
 (segment (start 147.795 75.105) (end 147.9 75) (width 1) (layer "F.Cu") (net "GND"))
 (segment (start 150.42 78.9) (end 150.7 79.18) (width 1) (layer "F.Cu") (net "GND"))
 (via (at 148 85.6) (size 0.6) (drill 0.3) (layers "F.Cu" "B.Cu") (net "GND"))
 (via (at 108.1 97.7) (size 0.6) (drill 0.3) (layers "F.Cu" "B.Cu") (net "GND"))
 (via (at 103.2 97.5) (size 0.6) (drill 0.3) (layers "F.Cu" "B.Cu") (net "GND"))
 (via (at 147.9 75) (size 0.6) (drill 0.3) (layers "F.Cu" "B.Cu") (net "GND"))
 (segment (start 147.033679 75) (end 147.9 75) (width 1) (layer "B.Cu") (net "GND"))
 (segment (start 146.733679 85.6) (end 143.755 82.621321) (width 1) (layer "B.Cu") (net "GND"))
 (segment (start 103.2 97.5) (end 107.9 97.5) (width 1) (layer "B.Cu") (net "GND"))
 (segment (start 148 85.6) (end 146.733679 85.6) (width 1) (layer "B.Cu") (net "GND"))
 (segment (start 143.755 78.278679) (end 147.033679 75) (width 1) (layer "B.Cu") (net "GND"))
 (segment (start 107.9 97.5) (end 108.1 97.7) (width 1) (layer "B.Cu") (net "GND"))
 (segment (start 143.755 82.621321) (end 143.755 78.278679) (width 1) (layer "B.Cu") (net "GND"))
 (segment (start 126.1 66.64) (end 117.86 66.64) (width 0.5) (layer "F.Cu") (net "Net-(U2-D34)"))
 (segment (start 126.5 66.24) (end 126.1 66.64) (width 0.5) (layer "F.Cu") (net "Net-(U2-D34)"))
 (segment (start 129.3 66.24) (end 126.5 66.24) (width 0.5) (layer "F.Cu") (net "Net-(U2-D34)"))
 (segment (start 117.86 66.64) (end 116.3 68.2) (width 0.5) (layer "F.Cu") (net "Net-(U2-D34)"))
 (segment (start 116.3 80.47) (end 118.825 82.995) (width 0.5) (layer "F.Cu") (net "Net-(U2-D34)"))
 (segment (start 116.3 68.2) (end 116.3 80.47) (width 0.5) (layer "F.Cu") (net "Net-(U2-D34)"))
 (segment (start 113.64 83.2) (end 113.64 81.28) (width 0.5) (layer "F.Cu") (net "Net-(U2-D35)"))
 (segment (start 118.825 85.535) (end 116.49 83.2) (width 0.5) (layer "F.Cu") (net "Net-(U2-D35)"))
 (segment (start 113.64 81.28) (end 111.16 78.8) (width 0.5) (layer "F.Cu") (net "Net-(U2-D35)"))
 (segment (start 116.49 83.2) (end 113.64 83.2) (width 0.5) (layer "F.Cu") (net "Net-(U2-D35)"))
 (segment (start 153.4 85.5) (end 153.4 74.6) (width 1) (layer "F.Cu") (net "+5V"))
 (segment (start 108.1025 109.635) (end 105.1 106.6325) (width 1) (layer "F.Cu") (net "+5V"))
 (segment (start 115.5 110.935) (end 118.825 110.935) (width 1) (layer "F.Cu") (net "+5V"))
 (segment (start 107.7 79.18) (end 105.82 79.18) (width 1) (layer "F.Cu") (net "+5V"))
 (segment (start 150.7 86.8) (end 152.1 86.8) (width 1) (layer "F.Cu") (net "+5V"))
 (segment (start 139.4 60.6) (end 134.3 60.6) (width 1) (layer "F.Cu") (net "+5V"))
 (segment (start 142.6 114.2) (end 150.7 106.1) (width 1) (layer "F.Cu") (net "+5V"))
 (segment (start 150.7 106.1) (end 150.7 86.8) (width 1) (layer "F.Cu") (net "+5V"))
 (segment (start 108.1025 109.635) (end 109.4025 110.935) (width 1) (layer "F.Cu") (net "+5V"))
 (segment (start 152.1 86.8) (end 153.4 85.5) (width 1) (layer "F.Cu") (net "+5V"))
 (segment (start 115.5 110.935) (end 115.5 111.7) (width 1) (layer "F.Cu") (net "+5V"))
 (segment (start 118 114.2) (end 142.6 114.2) (width 1) (layer "F.Cu") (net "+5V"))
 (segment (start 109.4025 110.935) (end 115.5 110.935) (width 1) (layer "F.Cu") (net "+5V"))
 (segment (start 105.1 79.9) (end 105.1 106.6325) (width 1) (layer "F.Cu") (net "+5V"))
 (segment (start 153.4 74.6) (end 139.4 60.6) (width 1) (layer "F.Cu") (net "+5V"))
 (segment (start 105.82 79.18) (end 105.1 79.9) (width 1) (layer "F.Cu") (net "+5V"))
 (segment (start 115.5 111.7) (end 118 114.2) (width 1) (layer "F.Cu") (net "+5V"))
 (segment (start 112.61 99.64) (end 118.825 105.855) (width 0.5) (layer "F.Cu") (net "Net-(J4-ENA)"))
 (segment (start 112 99.64) (end 112.61 99.64) (width 0.5) (layer "F.Cu") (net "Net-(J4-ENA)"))
 (segment (start 112 97.1) (end 115.675 100.775) (width 0.5) (layer "F.Cu") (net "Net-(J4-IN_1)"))
 (segment (start 115.675 100.775) (end 118.825 100.775) (width 0.5) (layer "F.Cu") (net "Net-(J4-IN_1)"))
 (segment (start 115.675 98.235) (end 118.825 98.235) (width 0.5) (layer "F.Cu") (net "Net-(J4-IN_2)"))
 (segment (start 112 94.56) (end 115.675 98.235) (width 0.5) (layer "F.Cu") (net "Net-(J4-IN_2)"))
 (segment (start 112 92.02) (end 115.675 95.695) (width 0.5) (layer "F.Cu") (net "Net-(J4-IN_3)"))
 (segment (start 115.675 95.695) (end 118.825 95.695) (width 0.5) (layer "F.Cu") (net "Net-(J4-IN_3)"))
 (segment (start 115.675 93.155) (end 118.825 93.155) (width 0.5) (layer "F.Cu") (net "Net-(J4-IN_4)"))
 (segment (start 112 89.48) (end 115.675 93.155) (width 0.5) (layer "F.Cu") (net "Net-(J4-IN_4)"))
 (segment (start 115.675 90.615) (end 118.825 90.615) (width 0.5) (layer "F.Cu") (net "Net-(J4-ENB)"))
 (segment (start 112 86.94) (end 115.675 90.615) (width 0.5) (layer "F.Cu") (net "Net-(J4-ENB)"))
 (segment (start 112.3 81.1) (end 112.35 81.15) (width 0.5) (layer "F.Cu") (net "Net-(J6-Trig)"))
 (segment (start 108.32 81.1) (end 112.3 81.1) (width 0.5) (layer "F.Cu") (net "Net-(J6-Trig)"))
 (segment (start 112.35 81.15) (end 112.35 84.45) (width 0.5) (layer "F.Cu") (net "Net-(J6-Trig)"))
 (segment (start 115.95 85.2) (end 118.825 88.075) (width 0.5) (layer "F.Cu") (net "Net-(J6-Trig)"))
 (segment (start 113.1 85.2) (end 115.95 85.2) (width 0.5) (layer "F.Cu") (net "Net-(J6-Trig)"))
 (segment (start 112.35 84.45) (end 113.1 85.2) (width 0.5) (layer "F.Cu") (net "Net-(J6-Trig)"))
 (segment (start 107.7 81.72) (end 108.32 81.1) (width 0.5) (layer "F.Cu") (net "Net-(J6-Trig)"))
 (segment (start 142.865 85.535) (end 141.685 85.535) (width 0.5) (layer "F.Cu") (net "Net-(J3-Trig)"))
 (segment (start 150.7 84.26) (end 144.14 84.26) (width 0.5) (layer "F.Cu") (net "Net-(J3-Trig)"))
 (segment (start 144.14 84.26) (end 142.865 85.535) (width 0.5) (layer "F.Cu") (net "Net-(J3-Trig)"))
 (segment (start 145.255 82) (end 145.255 78.9) (width 0.5) (layer "F.Cu") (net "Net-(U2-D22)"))
 (segment (start 141.685 77.915) (end 144.27 77.915) (width 0.5) (layer "F.Cu") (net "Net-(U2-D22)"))
 (segment (start 144.27 77.915) (end 145.255 78.9) (width 0.5) (layer "F.Cu") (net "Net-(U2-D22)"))
 (segment (start 144.1 67.2) (end 140.9 64) (width 0.5) (layer "F.Cu") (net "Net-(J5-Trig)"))
 (segment (start 131.76 63.76) (end 131.76 60.6) (width 0.5) (layer "F.Cu") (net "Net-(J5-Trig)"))
 (segment (start 141.685 75.375) (end 142.725 75.375) (width 0.5) (layer "F.Cu") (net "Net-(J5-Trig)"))
 (segment (start 140.9 64) (end 132 64) (width 0.5) (layer "F.Cu") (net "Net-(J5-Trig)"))
 (segment (start 144.1 74) (end 144.1 67.2) (width 0.5) (layer "F.Cu") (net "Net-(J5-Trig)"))
 (segment (start 142.725 75.375) (end 144.1 74) (width 0.5) (layer "F.Cu") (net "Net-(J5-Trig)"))
 (segment (start 132 64) (end 131.76 63.76) (width 0.5) (layer "F.Cu") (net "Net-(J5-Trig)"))
 (segment (start 148.075 81.72) (end 147.795 82) (width 0.5) (layer "F.Cu") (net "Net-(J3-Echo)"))
 (segment (start 150.7 81.72) (end 148.075 81.72) (width 0.5) (layer "F.Cu") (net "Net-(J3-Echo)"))
 (segment (start 129.3 60.68) (end 129.22 60.6) (width 0.5) (layer "F.Cu") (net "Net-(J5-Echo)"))
 (segment (start 129.3 63.7) (end 129.3 60.68) (width 0.5) (layer "F.Cu") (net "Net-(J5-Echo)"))
 (segment (start 110.04 84.26) (end 111.1 83.2) (width 0.5) (layer "F.Cu") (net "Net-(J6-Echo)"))
 (segment (start 107.7 84.26) (end 110.04 84.26) (width 0.5) (layer "F.Cu") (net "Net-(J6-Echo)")))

